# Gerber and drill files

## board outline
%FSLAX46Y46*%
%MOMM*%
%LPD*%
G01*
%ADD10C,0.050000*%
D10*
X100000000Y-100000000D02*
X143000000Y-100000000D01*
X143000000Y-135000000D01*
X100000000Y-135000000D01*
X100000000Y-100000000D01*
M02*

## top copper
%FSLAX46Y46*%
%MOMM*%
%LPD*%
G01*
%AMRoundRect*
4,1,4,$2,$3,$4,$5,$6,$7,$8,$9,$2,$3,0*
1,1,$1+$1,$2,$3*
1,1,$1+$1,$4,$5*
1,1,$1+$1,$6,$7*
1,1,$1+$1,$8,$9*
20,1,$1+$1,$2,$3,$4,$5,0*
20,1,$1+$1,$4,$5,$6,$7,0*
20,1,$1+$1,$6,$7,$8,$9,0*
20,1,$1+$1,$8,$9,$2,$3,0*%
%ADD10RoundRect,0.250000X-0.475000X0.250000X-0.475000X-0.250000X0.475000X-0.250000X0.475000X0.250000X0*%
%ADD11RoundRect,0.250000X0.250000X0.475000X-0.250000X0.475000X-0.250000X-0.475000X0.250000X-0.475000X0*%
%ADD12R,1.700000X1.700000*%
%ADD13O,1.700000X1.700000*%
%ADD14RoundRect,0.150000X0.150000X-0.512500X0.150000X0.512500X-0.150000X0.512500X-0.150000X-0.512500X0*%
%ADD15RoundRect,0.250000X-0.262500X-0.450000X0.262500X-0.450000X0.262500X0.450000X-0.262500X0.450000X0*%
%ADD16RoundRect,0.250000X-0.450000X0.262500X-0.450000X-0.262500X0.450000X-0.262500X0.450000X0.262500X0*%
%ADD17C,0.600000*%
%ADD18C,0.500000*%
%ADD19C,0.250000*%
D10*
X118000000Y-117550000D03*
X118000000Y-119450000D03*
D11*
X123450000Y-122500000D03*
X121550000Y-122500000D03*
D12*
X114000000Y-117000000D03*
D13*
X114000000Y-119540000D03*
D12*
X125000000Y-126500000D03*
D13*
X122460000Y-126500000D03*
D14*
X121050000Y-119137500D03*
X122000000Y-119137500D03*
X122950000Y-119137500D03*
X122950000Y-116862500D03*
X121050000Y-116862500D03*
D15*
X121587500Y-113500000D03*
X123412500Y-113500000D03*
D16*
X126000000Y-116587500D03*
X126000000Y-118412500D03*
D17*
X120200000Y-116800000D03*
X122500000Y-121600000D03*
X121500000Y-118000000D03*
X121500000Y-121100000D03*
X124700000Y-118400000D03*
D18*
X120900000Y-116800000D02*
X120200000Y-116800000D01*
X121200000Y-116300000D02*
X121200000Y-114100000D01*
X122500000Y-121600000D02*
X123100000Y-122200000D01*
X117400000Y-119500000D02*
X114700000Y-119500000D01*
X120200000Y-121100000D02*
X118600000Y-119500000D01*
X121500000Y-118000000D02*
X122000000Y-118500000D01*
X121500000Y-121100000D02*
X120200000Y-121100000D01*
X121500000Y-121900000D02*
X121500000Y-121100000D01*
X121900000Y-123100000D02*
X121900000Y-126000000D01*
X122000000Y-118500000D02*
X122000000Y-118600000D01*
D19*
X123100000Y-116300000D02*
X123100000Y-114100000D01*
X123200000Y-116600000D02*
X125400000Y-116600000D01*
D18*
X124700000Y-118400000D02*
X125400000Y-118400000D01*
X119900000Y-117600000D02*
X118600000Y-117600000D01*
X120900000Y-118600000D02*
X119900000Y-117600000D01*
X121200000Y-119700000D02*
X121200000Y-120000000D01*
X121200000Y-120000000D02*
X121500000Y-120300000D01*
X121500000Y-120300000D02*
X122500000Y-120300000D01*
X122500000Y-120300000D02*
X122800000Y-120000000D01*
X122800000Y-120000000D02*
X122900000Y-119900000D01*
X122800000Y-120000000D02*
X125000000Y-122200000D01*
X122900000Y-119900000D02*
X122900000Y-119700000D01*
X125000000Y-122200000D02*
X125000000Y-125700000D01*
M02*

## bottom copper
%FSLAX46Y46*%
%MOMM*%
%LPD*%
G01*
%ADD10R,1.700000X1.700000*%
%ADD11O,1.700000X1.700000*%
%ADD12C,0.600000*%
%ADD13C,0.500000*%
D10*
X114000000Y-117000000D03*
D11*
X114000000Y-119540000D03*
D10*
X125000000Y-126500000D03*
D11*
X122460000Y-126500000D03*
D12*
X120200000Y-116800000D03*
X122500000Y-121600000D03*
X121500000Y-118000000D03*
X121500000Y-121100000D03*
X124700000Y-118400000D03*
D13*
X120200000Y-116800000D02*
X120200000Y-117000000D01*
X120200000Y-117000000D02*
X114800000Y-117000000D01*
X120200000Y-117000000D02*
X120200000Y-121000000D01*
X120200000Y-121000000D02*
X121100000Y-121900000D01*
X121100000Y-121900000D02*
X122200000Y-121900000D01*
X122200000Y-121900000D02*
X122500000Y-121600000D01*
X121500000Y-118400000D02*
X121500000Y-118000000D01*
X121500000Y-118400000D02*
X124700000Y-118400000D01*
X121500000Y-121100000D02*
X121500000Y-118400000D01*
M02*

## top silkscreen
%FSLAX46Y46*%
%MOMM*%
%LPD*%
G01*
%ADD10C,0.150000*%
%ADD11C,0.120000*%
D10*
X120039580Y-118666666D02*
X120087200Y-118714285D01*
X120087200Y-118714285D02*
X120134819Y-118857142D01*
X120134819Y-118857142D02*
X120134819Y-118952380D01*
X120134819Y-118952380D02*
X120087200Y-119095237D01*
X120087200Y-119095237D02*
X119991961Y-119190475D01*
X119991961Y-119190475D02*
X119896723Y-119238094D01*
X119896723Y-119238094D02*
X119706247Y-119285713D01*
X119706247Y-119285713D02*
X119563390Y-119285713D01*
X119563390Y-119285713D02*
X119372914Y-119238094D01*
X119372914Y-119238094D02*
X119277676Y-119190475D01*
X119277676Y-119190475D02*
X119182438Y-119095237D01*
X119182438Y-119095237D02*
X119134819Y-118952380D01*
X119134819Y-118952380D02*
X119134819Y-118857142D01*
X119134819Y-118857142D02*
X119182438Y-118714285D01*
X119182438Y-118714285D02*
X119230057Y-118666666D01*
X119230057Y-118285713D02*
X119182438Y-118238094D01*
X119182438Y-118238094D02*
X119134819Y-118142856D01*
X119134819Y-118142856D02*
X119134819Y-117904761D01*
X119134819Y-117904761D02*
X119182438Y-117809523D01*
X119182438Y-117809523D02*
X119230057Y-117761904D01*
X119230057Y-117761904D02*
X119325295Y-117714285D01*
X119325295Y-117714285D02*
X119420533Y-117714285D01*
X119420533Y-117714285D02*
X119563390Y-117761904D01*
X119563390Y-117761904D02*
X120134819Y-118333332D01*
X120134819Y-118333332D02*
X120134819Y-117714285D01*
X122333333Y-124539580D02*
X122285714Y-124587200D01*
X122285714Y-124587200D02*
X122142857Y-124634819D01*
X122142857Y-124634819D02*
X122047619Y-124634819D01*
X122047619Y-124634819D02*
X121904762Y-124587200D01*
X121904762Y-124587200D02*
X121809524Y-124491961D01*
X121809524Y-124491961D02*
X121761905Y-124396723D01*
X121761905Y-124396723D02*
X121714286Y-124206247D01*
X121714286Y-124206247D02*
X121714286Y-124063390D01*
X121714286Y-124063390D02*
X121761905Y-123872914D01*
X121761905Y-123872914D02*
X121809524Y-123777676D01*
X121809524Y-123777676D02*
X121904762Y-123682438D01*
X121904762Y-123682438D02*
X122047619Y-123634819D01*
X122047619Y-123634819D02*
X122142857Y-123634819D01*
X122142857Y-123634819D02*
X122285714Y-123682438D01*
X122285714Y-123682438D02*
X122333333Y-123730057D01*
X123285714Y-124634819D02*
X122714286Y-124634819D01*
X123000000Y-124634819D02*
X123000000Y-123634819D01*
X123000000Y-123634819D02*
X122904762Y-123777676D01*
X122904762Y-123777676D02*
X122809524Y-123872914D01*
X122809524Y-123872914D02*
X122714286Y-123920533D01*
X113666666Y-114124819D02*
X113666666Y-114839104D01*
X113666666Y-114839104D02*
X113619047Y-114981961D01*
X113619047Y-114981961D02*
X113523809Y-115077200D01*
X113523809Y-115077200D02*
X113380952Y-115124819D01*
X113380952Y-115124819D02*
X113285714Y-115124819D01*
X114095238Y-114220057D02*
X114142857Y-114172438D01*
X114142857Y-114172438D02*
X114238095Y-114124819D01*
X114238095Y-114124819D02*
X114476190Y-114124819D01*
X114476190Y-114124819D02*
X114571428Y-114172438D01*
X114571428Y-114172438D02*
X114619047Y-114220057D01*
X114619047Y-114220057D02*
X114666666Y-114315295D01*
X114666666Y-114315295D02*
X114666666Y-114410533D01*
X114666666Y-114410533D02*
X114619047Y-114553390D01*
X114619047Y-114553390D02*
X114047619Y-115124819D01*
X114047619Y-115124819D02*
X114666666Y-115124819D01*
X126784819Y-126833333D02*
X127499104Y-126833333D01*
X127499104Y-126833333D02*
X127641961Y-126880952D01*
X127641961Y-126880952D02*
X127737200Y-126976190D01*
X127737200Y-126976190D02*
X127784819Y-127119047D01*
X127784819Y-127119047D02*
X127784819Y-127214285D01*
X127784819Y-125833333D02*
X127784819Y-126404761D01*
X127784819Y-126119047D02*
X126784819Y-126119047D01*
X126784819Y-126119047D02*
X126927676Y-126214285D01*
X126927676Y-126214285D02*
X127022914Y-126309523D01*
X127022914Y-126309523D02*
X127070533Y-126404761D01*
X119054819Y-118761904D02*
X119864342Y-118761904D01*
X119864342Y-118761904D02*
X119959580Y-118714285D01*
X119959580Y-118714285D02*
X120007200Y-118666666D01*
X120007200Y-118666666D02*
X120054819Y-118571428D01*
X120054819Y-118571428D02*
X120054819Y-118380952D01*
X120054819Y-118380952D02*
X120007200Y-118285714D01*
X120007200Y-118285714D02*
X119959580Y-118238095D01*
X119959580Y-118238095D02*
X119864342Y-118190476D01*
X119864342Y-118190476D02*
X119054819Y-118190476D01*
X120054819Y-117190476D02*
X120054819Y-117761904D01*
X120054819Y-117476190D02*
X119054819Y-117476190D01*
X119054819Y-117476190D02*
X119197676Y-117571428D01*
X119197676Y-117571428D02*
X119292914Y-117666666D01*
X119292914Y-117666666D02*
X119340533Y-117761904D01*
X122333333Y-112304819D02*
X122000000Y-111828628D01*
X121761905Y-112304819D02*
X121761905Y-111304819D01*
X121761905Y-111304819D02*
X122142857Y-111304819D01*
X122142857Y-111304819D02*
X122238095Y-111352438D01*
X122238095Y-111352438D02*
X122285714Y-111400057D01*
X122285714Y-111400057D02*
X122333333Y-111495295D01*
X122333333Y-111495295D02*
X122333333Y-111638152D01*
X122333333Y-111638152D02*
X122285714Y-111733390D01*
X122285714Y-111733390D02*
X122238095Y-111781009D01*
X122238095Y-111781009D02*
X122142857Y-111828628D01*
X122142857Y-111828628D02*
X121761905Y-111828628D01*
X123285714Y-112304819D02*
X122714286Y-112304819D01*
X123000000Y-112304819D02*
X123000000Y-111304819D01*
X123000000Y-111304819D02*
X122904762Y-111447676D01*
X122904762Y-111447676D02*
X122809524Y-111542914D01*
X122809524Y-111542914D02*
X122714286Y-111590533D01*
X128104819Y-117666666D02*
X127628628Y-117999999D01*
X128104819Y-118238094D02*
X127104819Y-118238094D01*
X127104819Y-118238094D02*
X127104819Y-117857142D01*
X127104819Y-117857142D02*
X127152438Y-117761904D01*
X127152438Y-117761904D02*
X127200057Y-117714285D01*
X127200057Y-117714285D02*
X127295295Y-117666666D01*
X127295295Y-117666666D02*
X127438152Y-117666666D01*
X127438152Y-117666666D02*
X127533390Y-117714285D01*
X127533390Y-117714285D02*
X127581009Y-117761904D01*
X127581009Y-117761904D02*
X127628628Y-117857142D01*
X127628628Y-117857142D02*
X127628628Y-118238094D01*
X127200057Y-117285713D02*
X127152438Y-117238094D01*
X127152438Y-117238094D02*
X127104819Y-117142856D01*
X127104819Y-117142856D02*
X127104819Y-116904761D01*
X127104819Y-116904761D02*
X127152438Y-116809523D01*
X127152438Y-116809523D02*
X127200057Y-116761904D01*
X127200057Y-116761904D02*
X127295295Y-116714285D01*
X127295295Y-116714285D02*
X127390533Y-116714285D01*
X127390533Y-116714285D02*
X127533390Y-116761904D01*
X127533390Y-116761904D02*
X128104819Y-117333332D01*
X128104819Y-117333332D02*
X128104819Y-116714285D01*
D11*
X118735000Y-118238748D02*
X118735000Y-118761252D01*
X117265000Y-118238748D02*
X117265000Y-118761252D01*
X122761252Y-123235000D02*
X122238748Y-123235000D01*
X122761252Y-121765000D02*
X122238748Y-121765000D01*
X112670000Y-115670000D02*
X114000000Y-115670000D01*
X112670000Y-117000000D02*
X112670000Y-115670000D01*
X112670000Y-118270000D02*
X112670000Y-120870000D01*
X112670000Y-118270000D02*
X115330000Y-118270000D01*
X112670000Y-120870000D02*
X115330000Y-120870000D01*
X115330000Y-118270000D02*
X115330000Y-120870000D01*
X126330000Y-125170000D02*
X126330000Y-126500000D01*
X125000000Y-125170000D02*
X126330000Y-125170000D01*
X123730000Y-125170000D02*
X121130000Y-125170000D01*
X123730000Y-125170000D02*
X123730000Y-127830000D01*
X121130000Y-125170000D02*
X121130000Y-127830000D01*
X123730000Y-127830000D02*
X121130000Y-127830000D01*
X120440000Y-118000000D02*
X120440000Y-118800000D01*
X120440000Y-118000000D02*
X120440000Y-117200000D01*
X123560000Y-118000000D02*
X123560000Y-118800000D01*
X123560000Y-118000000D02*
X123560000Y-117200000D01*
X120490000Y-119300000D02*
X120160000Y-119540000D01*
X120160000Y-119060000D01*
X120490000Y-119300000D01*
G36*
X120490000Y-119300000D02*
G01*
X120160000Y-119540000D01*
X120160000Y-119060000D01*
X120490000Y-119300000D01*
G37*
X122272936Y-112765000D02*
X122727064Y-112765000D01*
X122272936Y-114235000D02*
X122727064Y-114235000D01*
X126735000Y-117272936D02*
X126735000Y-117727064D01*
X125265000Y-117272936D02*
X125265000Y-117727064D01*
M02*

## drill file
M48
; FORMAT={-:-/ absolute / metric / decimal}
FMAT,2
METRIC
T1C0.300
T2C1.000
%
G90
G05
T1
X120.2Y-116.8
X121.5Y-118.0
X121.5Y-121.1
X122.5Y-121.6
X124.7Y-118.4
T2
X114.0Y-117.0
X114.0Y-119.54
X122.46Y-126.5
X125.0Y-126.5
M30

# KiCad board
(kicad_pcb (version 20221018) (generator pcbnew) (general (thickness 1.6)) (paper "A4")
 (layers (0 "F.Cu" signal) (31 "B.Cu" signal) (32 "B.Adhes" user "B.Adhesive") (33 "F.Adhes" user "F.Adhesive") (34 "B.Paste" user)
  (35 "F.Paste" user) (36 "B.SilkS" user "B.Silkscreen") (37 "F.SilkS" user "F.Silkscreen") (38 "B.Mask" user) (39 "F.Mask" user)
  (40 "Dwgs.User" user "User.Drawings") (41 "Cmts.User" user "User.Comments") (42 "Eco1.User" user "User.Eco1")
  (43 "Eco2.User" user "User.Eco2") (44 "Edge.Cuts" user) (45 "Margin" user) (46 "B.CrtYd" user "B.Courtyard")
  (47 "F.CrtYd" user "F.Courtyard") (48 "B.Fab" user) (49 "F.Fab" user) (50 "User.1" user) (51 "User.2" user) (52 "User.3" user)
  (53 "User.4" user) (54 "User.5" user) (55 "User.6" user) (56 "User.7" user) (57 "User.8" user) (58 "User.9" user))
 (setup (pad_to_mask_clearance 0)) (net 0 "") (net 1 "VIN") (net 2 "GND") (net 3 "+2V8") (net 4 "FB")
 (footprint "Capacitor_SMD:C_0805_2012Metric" (layer "F.Cu") (at 118 118.5 -90)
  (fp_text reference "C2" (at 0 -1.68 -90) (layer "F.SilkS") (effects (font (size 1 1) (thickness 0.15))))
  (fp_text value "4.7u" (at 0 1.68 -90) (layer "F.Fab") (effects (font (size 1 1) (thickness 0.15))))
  (fp_line (start -0.261252 -0.735) (end 0.261252 -0.735) (stroke (width 0.12) (type solid)) (layer "F.SilkS"))
  (fp_line (start -0.261252 0.735) (end 0.261252 0.735) (stroke (width 0.12) (type solid)) (layer "F.SilkS"))
  (pad "1" smd roundrect (at -0.95 0 270) (size 1 1.45) (layers "F.Cu" "F.Paste" "F.Mask") (roundrect_rratio 0.25) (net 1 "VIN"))
  (pad "2" smd roundrect (at 0.95 0 270) (size 1 1.45) (layers "F.Cu" "F.Paste" "F.Mask") (roundrect_rratio 0.25) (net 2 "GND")))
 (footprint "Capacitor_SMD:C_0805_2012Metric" (layer "F.Cu") (at 122.5 122.5 180)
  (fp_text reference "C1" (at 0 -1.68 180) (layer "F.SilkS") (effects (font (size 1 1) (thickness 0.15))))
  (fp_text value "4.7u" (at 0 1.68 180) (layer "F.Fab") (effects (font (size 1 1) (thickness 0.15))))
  (fp_line (start -0.261252 -0.735) (end 0.261252 -0.735) (stroke (width 0.12) (type solid)) (layer "F.SilkS"))
  (fp_line (start -0.261252 0.735) (end 0.261252 0.735) (stroke (width 0.12) (type solid)) (layer "F.SilkS"))
  (pad "1" smd roundrect (at -0.95 0 180) (size 1 1.45) (layers "F.Cu" "F.Paste" "F.Mask") (roundrect_rratio 0.25) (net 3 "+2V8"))
  (pad "2" smd roundrect (at 0.95 0 180) (size 1 1.45) (layers "F.Cu" "F.Paste" "F.Mask") (roundrect_rratio 0.25) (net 2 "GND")))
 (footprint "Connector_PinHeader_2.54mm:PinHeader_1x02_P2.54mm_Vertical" (layer "F.Cu") (at 114 117)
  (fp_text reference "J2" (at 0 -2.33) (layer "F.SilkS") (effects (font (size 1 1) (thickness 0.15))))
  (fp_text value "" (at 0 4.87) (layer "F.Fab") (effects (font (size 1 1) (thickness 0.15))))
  (fp_line (start -1.33 -1.33) (end 0 -1.33) (stroke (width 0.12) (type solid)) (layer "F.SilkS"))
  (fp_line (start -1.33 0) (end -1.33 -1.33) (stroke (width 0.12) (type solid)) (layer "F.SilkS"))
  (fp_line (start -1.33 1.27) (end -1.33 3.87) (stroke (width 0.12) (type solid)) (layer "F.SilkS"))
  (fp_line (start -1.33 1.27) (end 1.33 1.27) (stroke (width 0.12) (type solid)) (layer "F.SilkS"))
  (fp_line (start -1.33 3.87) (end 1.33 3.87) (stroke (width 0.12) (type solid)) (layer "F.SilkS"))
  (fp_line (start 1.33 1.27) (end 1.33 3.87) (stroke (width 0.12) (type solid)) (layer "F.SilkS"))
  (pad "1" thru_hole rect (at 0 0) (size 1.7 1.7) (drill 1) (layers "*.Cu" "*.Mask") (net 3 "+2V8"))
  (pad "2" thru_hole oval (at 0 2.54) (size 1.7 1.7) (drill 1) (layers "*.Cu" "*.Mask") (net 2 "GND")))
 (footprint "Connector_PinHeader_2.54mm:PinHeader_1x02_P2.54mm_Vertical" (layer "F.Cu") (at 125 126.5 -90)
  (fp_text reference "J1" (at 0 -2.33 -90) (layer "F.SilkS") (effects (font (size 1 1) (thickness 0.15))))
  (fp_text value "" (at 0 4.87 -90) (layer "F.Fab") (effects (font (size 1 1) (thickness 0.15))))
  (fp_line (start -1.33 -1.33) (end 0 -1.33) (stroke (width 0.12) (type solid)) (layer "F.SilkS"))
  (fp_line (start -1.33 0) (end -1.33 -1.33) (stroke (width 0.12) (type solid)) (layer "F.SilkS"))
  (fp_line (start -1.33 1.27) (end -1.33 3.87) (stroke (width 0.12) (type solid)) (layer "F.SilkS"))
  (fp_line (start -1.33 1.27) (end 1.33 1.27) (stroke (width 0.12) (type solid)) (layer "F.SilkS"))
  (fp_line (start -1.33 3.87) (end 1.33 3.87) (stroke (width 0.12) (type solid)) (layer "F.SilkS"))
  (fp_line (start 1.33 1.27) (end 1.33 3.87) (stroke (width 0.12) (type solid)) (layer "F.SilkS"))
  (pad "1" thru_hole rect (at 0 0 270) (size 1.7 1.7) (drill 1) (layers "*.Cu" "*.Mask") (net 1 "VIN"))
  (pad "2" thru_hole oval (at 0 2.54 270) (size 1.7 1.7) (drill 1) (layers "*.Cu" "*.Mask") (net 2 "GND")))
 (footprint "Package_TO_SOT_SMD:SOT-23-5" (layer "F.Cu") (at 122 118 90)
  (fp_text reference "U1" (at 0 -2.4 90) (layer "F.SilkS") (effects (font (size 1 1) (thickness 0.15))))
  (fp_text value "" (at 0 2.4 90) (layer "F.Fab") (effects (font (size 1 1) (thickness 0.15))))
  (fp_line (start 0 -1.56) (end -0.8 -1.56) (stroke (width 0.12) (type solid)) (layer "F.SilkS"))
  (fp_line (start 0 -1.56) (end 0.8 -1.56) (stroke (width 0.12) (type solid)) (layer "F.SilkS"))
  (fp_line (start 0 1.56) (end -0.8 1.56) (stroke (width 0.12) (type solid)) (layer "F.SilkS"))
  (fp_line (start 0 1.56) (end 0.8 1.56) (stroke (width 0.12) (type solid)) (layer "F.SilkS"))
  (fp_poly
   (pts (xy -1.3 -1.51) (xy -1.54 -1.84) (xy -1.06 -1.84) (xy -1.3 -1.51)) (stroke (width 0.12) (type solid)) (fill solid) (layer "F.SilkS"))
  (pad "1" smd roundrect (at -1.1375 -0.95 90) (size 1.325 0.6) (layers "F.Cu" "F.Paste" "F.Mask") (roundrect_rratio 0.25) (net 1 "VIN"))
  (pad "2" smd roundrect (at -1.1375 0 90) (size 1.325 0.6) (layers "F.Cu" "F.Paste" "F.Mask") (roundrect_rratio 0.25) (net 2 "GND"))
  (pad "3" smd roundrect (at -1.1375 0.95 90) (size 1.325 0.6) (layers "F.Cu" "F.Paste" "F.Mask") (roundrect_rratio 0.25) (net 1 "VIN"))
  (pad "4" smd roundrect (at 1.1375 0.95 90) (size 1.325 0.6) (layers "F.Cu" "F.Paste" "F.Mask") (roundrect_rratio 0.25) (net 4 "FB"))
  (pad "5" smd roundrect (at 1.1375 -0.95 90) (size 1.325 0.6) (layers "F.Cu" "F.Paste" "F.Mask") (roundrect_rratio 0.25) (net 3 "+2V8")))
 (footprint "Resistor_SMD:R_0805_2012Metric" (layer "F.Cu") (at 122.5 113.5)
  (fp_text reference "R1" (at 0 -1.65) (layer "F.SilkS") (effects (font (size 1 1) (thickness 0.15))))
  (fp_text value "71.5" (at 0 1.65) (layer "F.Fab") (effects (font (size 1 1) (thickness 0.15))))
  (fp_line (start -0.227064 -0.735) (end 0.227064 -0.735) (stroke (width 0.12) (type solid)) (layer "F.SilkS"))
  (fp_line (start -0.227064 0.735) (end 0.227064 0.735) (stroke (width 0.12) (type solid)) (layer "F.SilkS"))
  (pad "1" smd roundrect (at -0.9125 0) (size 1.025 1.4) (layers "F.Cu" "F.Paste" "F.Mask") (roundrect_rratio 0.243902) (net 3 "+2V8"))
  (pad "2" smd roundrect (at 0.9125 0) (size 1.025 1.4) (layers "F.Cu" "F.Paste" "F.Mask") (roundrect_rratio 0.243902) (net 4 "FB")))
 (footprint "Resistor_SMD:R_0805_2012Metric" (layer "F.Cu") (at 126 117.5 -90)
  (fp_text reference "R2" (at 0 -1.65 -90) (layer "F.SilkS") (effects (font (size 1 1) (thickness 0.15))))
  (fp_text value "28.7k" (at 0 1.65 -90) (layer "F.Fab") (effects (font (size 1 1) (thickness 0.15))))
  (fp_line (start -0.227064 -0.735) (end 0.227064 -0.735) (stroke (width 0.12) (type solid)) (layer "F.SilkS"))
  (fp_line (start -0.227064 0.735) (end 0.227064 0.735) (stroke (width 0.12) (type solid)) (layer "F.SilkS"))
  (pad "1" smd roundrect (at -0.9125 0 270) (size 1.025 1.4) (layers "F.Cu" "F.Paste" "F.Mask") (roundrect_rratio 0.243902) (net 4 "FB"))
  (pad "2" smd roundrect (at 0.9125 0 270) (size 1.025 1.4) (layers "F.Cu" "F.Paste" "F.Mask") (roundrect_rratio 0.243902) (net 2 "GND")))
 (gr_rect (start 100 100) (end 143 135) (stroke (width 0.05) (type default)) (fill none) (layer "Edge.Cuts"))
 (segment (start 120.9 116.8) (end 120.2 116.8) (width 0.5) (layer "F.Cu") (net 3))
 (segment (start 121.2 116.3) (end 121.2 114.1) (width 0.5) (layer "F.Cu") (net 3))
 (segment (start 122.5 121.6) (end 123.1 122.2) (width 0.5) (layer "F.Cu") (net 3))
 (via (at 120.2 116.8) (size 0.6) (drill 0.3) (layers "F.Cu" "B.Cu") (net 3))
 (via (at 122.5 121.6) (size 0.6) (drill 0.3) (layers "F.Cu" "B.Cu") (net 3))
 (segment (start 117.4 119.5) (end 114.7 119.5) (width 0.5) (layer "F.Cu") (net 2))
 (segment (start 120.2 116.8) (end 120.2 117) (width 0.5) (layer "B.Cu") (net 3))
 (segment (start 120.2 117) (end 114.8 117) (width 0.5) (layer "B.Cu") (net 3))
 (segment (start 120.2 117) (end 120.2 121) (width 0.5) (layer "B.Cu") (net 3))
 (segment (start 120.2 121) (end 121.1 121.9) (width 0.5) (layer "B.Cu") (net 3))
 (segment (start 120.2 121.1) (end 118.6 119.5) (width 0.5) (layer "F.Cu") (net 2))
 (segment (start 121.1 121.9) (end 122.2 121.9) (width 0.5) (layer "B.Cu") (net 3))
 (segment (start 121.5 118) (end 122 118.5) (width 0.5) (layer "F.Cu") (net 2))
 (segment (start 121.5 121.1) (end 120.2 121.1) (width 0.5) (layer "F.Cu") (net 2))
 (segment (start 121.5 121.9) (end 121.5 121.1) (width 0.5) (layer "F.Cu") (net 2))
 (segment (start 121.9 123.1) (end 121.9 126) (width 0.5) (layer "F.Cu") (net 2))
 (segment (start 122 118.5) (end 122 118.6) (width 0.5) (layer "F.Cu") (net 2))
 (segment (start 122.2 121.9) (end 122.5 121.6) (width 0.5) (layer "B.Cu") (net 3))
 (segment (start 123.1 116.3) (end 123.1 114.1) (width 0.25) (layer "F.Cu") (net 4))
 (segment (start 123.2 116.6) (end 125.4 116.6) (width 0.25) (layer "F.Cu") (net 4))
 (segment (start 124.7 118.4) (end 125.4 118.4) (width 0.5) (layer "F.Cu") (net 2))
 (via (at 121.5 118) (size 0.6) (drill 0.3) (layers "F.Cu" "B.Cu") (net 2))
 (via (at 121.5 121.1) (size 0.6) (drill 0.3) (layers "F.Cu" "B.Cu") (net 2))
 (via (at 124.7 118.4) (size 0.6) (drill 0.3) (layers "F.Cu" "B.Cu") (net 2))
 (segment (start 119.9 117.6) (end 118.6 117.6) (width 0.5) (layer "F.Cu") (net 1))
 (segment (start 120.9 118.6) (end 119.9 117.6) (width 0.5) (layer "F.Cu") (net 1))
 (segment (start 121.2 119.7) (end 121.2 120) (width 0.5) (layer "F.Cu") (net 1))
 (segment (start 121.2 120) (end 121.5 120.3) (width 0.5) (layer "F.Cu") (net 1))
 (segment (start 121.5 118.4) (end 121.5 118) (width 0.5) (layer "B.Cu") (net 2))
 (segment (start 121.5 118.4) (end 124.7 118.4) (width 0.5) (layer "B.Cu") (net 2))
 (segment (start 121.5 120.3) (end 122.5 120.3) (width 0.5) (layer "F.Cu") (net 1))
 (segment (start 121.5 121.1) (end 121.5 118.4) (width 0.5) (layer "B.Cu") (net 2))
 (segment (start 122.5 120.3) (end 122.8 120) (width 0.5) (layer "F.Cu") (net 1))
 (segment (start 122.8 120) (end 122.9 119.9) (width 0.5) (layer "F.Cu") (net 1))
 (segment (start 122.8 120) (end 125 122.2) (width 0.5) (layer "F.Cu") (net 1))
 (segment (start 122.9 119.9) (end 122.9 119.7) (width 0.5) (layer "F.Cu") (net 1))
 (segment (start 125 122.2) (end 125 125.7) (width 0.5) (layer "F.Cu") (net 1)))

